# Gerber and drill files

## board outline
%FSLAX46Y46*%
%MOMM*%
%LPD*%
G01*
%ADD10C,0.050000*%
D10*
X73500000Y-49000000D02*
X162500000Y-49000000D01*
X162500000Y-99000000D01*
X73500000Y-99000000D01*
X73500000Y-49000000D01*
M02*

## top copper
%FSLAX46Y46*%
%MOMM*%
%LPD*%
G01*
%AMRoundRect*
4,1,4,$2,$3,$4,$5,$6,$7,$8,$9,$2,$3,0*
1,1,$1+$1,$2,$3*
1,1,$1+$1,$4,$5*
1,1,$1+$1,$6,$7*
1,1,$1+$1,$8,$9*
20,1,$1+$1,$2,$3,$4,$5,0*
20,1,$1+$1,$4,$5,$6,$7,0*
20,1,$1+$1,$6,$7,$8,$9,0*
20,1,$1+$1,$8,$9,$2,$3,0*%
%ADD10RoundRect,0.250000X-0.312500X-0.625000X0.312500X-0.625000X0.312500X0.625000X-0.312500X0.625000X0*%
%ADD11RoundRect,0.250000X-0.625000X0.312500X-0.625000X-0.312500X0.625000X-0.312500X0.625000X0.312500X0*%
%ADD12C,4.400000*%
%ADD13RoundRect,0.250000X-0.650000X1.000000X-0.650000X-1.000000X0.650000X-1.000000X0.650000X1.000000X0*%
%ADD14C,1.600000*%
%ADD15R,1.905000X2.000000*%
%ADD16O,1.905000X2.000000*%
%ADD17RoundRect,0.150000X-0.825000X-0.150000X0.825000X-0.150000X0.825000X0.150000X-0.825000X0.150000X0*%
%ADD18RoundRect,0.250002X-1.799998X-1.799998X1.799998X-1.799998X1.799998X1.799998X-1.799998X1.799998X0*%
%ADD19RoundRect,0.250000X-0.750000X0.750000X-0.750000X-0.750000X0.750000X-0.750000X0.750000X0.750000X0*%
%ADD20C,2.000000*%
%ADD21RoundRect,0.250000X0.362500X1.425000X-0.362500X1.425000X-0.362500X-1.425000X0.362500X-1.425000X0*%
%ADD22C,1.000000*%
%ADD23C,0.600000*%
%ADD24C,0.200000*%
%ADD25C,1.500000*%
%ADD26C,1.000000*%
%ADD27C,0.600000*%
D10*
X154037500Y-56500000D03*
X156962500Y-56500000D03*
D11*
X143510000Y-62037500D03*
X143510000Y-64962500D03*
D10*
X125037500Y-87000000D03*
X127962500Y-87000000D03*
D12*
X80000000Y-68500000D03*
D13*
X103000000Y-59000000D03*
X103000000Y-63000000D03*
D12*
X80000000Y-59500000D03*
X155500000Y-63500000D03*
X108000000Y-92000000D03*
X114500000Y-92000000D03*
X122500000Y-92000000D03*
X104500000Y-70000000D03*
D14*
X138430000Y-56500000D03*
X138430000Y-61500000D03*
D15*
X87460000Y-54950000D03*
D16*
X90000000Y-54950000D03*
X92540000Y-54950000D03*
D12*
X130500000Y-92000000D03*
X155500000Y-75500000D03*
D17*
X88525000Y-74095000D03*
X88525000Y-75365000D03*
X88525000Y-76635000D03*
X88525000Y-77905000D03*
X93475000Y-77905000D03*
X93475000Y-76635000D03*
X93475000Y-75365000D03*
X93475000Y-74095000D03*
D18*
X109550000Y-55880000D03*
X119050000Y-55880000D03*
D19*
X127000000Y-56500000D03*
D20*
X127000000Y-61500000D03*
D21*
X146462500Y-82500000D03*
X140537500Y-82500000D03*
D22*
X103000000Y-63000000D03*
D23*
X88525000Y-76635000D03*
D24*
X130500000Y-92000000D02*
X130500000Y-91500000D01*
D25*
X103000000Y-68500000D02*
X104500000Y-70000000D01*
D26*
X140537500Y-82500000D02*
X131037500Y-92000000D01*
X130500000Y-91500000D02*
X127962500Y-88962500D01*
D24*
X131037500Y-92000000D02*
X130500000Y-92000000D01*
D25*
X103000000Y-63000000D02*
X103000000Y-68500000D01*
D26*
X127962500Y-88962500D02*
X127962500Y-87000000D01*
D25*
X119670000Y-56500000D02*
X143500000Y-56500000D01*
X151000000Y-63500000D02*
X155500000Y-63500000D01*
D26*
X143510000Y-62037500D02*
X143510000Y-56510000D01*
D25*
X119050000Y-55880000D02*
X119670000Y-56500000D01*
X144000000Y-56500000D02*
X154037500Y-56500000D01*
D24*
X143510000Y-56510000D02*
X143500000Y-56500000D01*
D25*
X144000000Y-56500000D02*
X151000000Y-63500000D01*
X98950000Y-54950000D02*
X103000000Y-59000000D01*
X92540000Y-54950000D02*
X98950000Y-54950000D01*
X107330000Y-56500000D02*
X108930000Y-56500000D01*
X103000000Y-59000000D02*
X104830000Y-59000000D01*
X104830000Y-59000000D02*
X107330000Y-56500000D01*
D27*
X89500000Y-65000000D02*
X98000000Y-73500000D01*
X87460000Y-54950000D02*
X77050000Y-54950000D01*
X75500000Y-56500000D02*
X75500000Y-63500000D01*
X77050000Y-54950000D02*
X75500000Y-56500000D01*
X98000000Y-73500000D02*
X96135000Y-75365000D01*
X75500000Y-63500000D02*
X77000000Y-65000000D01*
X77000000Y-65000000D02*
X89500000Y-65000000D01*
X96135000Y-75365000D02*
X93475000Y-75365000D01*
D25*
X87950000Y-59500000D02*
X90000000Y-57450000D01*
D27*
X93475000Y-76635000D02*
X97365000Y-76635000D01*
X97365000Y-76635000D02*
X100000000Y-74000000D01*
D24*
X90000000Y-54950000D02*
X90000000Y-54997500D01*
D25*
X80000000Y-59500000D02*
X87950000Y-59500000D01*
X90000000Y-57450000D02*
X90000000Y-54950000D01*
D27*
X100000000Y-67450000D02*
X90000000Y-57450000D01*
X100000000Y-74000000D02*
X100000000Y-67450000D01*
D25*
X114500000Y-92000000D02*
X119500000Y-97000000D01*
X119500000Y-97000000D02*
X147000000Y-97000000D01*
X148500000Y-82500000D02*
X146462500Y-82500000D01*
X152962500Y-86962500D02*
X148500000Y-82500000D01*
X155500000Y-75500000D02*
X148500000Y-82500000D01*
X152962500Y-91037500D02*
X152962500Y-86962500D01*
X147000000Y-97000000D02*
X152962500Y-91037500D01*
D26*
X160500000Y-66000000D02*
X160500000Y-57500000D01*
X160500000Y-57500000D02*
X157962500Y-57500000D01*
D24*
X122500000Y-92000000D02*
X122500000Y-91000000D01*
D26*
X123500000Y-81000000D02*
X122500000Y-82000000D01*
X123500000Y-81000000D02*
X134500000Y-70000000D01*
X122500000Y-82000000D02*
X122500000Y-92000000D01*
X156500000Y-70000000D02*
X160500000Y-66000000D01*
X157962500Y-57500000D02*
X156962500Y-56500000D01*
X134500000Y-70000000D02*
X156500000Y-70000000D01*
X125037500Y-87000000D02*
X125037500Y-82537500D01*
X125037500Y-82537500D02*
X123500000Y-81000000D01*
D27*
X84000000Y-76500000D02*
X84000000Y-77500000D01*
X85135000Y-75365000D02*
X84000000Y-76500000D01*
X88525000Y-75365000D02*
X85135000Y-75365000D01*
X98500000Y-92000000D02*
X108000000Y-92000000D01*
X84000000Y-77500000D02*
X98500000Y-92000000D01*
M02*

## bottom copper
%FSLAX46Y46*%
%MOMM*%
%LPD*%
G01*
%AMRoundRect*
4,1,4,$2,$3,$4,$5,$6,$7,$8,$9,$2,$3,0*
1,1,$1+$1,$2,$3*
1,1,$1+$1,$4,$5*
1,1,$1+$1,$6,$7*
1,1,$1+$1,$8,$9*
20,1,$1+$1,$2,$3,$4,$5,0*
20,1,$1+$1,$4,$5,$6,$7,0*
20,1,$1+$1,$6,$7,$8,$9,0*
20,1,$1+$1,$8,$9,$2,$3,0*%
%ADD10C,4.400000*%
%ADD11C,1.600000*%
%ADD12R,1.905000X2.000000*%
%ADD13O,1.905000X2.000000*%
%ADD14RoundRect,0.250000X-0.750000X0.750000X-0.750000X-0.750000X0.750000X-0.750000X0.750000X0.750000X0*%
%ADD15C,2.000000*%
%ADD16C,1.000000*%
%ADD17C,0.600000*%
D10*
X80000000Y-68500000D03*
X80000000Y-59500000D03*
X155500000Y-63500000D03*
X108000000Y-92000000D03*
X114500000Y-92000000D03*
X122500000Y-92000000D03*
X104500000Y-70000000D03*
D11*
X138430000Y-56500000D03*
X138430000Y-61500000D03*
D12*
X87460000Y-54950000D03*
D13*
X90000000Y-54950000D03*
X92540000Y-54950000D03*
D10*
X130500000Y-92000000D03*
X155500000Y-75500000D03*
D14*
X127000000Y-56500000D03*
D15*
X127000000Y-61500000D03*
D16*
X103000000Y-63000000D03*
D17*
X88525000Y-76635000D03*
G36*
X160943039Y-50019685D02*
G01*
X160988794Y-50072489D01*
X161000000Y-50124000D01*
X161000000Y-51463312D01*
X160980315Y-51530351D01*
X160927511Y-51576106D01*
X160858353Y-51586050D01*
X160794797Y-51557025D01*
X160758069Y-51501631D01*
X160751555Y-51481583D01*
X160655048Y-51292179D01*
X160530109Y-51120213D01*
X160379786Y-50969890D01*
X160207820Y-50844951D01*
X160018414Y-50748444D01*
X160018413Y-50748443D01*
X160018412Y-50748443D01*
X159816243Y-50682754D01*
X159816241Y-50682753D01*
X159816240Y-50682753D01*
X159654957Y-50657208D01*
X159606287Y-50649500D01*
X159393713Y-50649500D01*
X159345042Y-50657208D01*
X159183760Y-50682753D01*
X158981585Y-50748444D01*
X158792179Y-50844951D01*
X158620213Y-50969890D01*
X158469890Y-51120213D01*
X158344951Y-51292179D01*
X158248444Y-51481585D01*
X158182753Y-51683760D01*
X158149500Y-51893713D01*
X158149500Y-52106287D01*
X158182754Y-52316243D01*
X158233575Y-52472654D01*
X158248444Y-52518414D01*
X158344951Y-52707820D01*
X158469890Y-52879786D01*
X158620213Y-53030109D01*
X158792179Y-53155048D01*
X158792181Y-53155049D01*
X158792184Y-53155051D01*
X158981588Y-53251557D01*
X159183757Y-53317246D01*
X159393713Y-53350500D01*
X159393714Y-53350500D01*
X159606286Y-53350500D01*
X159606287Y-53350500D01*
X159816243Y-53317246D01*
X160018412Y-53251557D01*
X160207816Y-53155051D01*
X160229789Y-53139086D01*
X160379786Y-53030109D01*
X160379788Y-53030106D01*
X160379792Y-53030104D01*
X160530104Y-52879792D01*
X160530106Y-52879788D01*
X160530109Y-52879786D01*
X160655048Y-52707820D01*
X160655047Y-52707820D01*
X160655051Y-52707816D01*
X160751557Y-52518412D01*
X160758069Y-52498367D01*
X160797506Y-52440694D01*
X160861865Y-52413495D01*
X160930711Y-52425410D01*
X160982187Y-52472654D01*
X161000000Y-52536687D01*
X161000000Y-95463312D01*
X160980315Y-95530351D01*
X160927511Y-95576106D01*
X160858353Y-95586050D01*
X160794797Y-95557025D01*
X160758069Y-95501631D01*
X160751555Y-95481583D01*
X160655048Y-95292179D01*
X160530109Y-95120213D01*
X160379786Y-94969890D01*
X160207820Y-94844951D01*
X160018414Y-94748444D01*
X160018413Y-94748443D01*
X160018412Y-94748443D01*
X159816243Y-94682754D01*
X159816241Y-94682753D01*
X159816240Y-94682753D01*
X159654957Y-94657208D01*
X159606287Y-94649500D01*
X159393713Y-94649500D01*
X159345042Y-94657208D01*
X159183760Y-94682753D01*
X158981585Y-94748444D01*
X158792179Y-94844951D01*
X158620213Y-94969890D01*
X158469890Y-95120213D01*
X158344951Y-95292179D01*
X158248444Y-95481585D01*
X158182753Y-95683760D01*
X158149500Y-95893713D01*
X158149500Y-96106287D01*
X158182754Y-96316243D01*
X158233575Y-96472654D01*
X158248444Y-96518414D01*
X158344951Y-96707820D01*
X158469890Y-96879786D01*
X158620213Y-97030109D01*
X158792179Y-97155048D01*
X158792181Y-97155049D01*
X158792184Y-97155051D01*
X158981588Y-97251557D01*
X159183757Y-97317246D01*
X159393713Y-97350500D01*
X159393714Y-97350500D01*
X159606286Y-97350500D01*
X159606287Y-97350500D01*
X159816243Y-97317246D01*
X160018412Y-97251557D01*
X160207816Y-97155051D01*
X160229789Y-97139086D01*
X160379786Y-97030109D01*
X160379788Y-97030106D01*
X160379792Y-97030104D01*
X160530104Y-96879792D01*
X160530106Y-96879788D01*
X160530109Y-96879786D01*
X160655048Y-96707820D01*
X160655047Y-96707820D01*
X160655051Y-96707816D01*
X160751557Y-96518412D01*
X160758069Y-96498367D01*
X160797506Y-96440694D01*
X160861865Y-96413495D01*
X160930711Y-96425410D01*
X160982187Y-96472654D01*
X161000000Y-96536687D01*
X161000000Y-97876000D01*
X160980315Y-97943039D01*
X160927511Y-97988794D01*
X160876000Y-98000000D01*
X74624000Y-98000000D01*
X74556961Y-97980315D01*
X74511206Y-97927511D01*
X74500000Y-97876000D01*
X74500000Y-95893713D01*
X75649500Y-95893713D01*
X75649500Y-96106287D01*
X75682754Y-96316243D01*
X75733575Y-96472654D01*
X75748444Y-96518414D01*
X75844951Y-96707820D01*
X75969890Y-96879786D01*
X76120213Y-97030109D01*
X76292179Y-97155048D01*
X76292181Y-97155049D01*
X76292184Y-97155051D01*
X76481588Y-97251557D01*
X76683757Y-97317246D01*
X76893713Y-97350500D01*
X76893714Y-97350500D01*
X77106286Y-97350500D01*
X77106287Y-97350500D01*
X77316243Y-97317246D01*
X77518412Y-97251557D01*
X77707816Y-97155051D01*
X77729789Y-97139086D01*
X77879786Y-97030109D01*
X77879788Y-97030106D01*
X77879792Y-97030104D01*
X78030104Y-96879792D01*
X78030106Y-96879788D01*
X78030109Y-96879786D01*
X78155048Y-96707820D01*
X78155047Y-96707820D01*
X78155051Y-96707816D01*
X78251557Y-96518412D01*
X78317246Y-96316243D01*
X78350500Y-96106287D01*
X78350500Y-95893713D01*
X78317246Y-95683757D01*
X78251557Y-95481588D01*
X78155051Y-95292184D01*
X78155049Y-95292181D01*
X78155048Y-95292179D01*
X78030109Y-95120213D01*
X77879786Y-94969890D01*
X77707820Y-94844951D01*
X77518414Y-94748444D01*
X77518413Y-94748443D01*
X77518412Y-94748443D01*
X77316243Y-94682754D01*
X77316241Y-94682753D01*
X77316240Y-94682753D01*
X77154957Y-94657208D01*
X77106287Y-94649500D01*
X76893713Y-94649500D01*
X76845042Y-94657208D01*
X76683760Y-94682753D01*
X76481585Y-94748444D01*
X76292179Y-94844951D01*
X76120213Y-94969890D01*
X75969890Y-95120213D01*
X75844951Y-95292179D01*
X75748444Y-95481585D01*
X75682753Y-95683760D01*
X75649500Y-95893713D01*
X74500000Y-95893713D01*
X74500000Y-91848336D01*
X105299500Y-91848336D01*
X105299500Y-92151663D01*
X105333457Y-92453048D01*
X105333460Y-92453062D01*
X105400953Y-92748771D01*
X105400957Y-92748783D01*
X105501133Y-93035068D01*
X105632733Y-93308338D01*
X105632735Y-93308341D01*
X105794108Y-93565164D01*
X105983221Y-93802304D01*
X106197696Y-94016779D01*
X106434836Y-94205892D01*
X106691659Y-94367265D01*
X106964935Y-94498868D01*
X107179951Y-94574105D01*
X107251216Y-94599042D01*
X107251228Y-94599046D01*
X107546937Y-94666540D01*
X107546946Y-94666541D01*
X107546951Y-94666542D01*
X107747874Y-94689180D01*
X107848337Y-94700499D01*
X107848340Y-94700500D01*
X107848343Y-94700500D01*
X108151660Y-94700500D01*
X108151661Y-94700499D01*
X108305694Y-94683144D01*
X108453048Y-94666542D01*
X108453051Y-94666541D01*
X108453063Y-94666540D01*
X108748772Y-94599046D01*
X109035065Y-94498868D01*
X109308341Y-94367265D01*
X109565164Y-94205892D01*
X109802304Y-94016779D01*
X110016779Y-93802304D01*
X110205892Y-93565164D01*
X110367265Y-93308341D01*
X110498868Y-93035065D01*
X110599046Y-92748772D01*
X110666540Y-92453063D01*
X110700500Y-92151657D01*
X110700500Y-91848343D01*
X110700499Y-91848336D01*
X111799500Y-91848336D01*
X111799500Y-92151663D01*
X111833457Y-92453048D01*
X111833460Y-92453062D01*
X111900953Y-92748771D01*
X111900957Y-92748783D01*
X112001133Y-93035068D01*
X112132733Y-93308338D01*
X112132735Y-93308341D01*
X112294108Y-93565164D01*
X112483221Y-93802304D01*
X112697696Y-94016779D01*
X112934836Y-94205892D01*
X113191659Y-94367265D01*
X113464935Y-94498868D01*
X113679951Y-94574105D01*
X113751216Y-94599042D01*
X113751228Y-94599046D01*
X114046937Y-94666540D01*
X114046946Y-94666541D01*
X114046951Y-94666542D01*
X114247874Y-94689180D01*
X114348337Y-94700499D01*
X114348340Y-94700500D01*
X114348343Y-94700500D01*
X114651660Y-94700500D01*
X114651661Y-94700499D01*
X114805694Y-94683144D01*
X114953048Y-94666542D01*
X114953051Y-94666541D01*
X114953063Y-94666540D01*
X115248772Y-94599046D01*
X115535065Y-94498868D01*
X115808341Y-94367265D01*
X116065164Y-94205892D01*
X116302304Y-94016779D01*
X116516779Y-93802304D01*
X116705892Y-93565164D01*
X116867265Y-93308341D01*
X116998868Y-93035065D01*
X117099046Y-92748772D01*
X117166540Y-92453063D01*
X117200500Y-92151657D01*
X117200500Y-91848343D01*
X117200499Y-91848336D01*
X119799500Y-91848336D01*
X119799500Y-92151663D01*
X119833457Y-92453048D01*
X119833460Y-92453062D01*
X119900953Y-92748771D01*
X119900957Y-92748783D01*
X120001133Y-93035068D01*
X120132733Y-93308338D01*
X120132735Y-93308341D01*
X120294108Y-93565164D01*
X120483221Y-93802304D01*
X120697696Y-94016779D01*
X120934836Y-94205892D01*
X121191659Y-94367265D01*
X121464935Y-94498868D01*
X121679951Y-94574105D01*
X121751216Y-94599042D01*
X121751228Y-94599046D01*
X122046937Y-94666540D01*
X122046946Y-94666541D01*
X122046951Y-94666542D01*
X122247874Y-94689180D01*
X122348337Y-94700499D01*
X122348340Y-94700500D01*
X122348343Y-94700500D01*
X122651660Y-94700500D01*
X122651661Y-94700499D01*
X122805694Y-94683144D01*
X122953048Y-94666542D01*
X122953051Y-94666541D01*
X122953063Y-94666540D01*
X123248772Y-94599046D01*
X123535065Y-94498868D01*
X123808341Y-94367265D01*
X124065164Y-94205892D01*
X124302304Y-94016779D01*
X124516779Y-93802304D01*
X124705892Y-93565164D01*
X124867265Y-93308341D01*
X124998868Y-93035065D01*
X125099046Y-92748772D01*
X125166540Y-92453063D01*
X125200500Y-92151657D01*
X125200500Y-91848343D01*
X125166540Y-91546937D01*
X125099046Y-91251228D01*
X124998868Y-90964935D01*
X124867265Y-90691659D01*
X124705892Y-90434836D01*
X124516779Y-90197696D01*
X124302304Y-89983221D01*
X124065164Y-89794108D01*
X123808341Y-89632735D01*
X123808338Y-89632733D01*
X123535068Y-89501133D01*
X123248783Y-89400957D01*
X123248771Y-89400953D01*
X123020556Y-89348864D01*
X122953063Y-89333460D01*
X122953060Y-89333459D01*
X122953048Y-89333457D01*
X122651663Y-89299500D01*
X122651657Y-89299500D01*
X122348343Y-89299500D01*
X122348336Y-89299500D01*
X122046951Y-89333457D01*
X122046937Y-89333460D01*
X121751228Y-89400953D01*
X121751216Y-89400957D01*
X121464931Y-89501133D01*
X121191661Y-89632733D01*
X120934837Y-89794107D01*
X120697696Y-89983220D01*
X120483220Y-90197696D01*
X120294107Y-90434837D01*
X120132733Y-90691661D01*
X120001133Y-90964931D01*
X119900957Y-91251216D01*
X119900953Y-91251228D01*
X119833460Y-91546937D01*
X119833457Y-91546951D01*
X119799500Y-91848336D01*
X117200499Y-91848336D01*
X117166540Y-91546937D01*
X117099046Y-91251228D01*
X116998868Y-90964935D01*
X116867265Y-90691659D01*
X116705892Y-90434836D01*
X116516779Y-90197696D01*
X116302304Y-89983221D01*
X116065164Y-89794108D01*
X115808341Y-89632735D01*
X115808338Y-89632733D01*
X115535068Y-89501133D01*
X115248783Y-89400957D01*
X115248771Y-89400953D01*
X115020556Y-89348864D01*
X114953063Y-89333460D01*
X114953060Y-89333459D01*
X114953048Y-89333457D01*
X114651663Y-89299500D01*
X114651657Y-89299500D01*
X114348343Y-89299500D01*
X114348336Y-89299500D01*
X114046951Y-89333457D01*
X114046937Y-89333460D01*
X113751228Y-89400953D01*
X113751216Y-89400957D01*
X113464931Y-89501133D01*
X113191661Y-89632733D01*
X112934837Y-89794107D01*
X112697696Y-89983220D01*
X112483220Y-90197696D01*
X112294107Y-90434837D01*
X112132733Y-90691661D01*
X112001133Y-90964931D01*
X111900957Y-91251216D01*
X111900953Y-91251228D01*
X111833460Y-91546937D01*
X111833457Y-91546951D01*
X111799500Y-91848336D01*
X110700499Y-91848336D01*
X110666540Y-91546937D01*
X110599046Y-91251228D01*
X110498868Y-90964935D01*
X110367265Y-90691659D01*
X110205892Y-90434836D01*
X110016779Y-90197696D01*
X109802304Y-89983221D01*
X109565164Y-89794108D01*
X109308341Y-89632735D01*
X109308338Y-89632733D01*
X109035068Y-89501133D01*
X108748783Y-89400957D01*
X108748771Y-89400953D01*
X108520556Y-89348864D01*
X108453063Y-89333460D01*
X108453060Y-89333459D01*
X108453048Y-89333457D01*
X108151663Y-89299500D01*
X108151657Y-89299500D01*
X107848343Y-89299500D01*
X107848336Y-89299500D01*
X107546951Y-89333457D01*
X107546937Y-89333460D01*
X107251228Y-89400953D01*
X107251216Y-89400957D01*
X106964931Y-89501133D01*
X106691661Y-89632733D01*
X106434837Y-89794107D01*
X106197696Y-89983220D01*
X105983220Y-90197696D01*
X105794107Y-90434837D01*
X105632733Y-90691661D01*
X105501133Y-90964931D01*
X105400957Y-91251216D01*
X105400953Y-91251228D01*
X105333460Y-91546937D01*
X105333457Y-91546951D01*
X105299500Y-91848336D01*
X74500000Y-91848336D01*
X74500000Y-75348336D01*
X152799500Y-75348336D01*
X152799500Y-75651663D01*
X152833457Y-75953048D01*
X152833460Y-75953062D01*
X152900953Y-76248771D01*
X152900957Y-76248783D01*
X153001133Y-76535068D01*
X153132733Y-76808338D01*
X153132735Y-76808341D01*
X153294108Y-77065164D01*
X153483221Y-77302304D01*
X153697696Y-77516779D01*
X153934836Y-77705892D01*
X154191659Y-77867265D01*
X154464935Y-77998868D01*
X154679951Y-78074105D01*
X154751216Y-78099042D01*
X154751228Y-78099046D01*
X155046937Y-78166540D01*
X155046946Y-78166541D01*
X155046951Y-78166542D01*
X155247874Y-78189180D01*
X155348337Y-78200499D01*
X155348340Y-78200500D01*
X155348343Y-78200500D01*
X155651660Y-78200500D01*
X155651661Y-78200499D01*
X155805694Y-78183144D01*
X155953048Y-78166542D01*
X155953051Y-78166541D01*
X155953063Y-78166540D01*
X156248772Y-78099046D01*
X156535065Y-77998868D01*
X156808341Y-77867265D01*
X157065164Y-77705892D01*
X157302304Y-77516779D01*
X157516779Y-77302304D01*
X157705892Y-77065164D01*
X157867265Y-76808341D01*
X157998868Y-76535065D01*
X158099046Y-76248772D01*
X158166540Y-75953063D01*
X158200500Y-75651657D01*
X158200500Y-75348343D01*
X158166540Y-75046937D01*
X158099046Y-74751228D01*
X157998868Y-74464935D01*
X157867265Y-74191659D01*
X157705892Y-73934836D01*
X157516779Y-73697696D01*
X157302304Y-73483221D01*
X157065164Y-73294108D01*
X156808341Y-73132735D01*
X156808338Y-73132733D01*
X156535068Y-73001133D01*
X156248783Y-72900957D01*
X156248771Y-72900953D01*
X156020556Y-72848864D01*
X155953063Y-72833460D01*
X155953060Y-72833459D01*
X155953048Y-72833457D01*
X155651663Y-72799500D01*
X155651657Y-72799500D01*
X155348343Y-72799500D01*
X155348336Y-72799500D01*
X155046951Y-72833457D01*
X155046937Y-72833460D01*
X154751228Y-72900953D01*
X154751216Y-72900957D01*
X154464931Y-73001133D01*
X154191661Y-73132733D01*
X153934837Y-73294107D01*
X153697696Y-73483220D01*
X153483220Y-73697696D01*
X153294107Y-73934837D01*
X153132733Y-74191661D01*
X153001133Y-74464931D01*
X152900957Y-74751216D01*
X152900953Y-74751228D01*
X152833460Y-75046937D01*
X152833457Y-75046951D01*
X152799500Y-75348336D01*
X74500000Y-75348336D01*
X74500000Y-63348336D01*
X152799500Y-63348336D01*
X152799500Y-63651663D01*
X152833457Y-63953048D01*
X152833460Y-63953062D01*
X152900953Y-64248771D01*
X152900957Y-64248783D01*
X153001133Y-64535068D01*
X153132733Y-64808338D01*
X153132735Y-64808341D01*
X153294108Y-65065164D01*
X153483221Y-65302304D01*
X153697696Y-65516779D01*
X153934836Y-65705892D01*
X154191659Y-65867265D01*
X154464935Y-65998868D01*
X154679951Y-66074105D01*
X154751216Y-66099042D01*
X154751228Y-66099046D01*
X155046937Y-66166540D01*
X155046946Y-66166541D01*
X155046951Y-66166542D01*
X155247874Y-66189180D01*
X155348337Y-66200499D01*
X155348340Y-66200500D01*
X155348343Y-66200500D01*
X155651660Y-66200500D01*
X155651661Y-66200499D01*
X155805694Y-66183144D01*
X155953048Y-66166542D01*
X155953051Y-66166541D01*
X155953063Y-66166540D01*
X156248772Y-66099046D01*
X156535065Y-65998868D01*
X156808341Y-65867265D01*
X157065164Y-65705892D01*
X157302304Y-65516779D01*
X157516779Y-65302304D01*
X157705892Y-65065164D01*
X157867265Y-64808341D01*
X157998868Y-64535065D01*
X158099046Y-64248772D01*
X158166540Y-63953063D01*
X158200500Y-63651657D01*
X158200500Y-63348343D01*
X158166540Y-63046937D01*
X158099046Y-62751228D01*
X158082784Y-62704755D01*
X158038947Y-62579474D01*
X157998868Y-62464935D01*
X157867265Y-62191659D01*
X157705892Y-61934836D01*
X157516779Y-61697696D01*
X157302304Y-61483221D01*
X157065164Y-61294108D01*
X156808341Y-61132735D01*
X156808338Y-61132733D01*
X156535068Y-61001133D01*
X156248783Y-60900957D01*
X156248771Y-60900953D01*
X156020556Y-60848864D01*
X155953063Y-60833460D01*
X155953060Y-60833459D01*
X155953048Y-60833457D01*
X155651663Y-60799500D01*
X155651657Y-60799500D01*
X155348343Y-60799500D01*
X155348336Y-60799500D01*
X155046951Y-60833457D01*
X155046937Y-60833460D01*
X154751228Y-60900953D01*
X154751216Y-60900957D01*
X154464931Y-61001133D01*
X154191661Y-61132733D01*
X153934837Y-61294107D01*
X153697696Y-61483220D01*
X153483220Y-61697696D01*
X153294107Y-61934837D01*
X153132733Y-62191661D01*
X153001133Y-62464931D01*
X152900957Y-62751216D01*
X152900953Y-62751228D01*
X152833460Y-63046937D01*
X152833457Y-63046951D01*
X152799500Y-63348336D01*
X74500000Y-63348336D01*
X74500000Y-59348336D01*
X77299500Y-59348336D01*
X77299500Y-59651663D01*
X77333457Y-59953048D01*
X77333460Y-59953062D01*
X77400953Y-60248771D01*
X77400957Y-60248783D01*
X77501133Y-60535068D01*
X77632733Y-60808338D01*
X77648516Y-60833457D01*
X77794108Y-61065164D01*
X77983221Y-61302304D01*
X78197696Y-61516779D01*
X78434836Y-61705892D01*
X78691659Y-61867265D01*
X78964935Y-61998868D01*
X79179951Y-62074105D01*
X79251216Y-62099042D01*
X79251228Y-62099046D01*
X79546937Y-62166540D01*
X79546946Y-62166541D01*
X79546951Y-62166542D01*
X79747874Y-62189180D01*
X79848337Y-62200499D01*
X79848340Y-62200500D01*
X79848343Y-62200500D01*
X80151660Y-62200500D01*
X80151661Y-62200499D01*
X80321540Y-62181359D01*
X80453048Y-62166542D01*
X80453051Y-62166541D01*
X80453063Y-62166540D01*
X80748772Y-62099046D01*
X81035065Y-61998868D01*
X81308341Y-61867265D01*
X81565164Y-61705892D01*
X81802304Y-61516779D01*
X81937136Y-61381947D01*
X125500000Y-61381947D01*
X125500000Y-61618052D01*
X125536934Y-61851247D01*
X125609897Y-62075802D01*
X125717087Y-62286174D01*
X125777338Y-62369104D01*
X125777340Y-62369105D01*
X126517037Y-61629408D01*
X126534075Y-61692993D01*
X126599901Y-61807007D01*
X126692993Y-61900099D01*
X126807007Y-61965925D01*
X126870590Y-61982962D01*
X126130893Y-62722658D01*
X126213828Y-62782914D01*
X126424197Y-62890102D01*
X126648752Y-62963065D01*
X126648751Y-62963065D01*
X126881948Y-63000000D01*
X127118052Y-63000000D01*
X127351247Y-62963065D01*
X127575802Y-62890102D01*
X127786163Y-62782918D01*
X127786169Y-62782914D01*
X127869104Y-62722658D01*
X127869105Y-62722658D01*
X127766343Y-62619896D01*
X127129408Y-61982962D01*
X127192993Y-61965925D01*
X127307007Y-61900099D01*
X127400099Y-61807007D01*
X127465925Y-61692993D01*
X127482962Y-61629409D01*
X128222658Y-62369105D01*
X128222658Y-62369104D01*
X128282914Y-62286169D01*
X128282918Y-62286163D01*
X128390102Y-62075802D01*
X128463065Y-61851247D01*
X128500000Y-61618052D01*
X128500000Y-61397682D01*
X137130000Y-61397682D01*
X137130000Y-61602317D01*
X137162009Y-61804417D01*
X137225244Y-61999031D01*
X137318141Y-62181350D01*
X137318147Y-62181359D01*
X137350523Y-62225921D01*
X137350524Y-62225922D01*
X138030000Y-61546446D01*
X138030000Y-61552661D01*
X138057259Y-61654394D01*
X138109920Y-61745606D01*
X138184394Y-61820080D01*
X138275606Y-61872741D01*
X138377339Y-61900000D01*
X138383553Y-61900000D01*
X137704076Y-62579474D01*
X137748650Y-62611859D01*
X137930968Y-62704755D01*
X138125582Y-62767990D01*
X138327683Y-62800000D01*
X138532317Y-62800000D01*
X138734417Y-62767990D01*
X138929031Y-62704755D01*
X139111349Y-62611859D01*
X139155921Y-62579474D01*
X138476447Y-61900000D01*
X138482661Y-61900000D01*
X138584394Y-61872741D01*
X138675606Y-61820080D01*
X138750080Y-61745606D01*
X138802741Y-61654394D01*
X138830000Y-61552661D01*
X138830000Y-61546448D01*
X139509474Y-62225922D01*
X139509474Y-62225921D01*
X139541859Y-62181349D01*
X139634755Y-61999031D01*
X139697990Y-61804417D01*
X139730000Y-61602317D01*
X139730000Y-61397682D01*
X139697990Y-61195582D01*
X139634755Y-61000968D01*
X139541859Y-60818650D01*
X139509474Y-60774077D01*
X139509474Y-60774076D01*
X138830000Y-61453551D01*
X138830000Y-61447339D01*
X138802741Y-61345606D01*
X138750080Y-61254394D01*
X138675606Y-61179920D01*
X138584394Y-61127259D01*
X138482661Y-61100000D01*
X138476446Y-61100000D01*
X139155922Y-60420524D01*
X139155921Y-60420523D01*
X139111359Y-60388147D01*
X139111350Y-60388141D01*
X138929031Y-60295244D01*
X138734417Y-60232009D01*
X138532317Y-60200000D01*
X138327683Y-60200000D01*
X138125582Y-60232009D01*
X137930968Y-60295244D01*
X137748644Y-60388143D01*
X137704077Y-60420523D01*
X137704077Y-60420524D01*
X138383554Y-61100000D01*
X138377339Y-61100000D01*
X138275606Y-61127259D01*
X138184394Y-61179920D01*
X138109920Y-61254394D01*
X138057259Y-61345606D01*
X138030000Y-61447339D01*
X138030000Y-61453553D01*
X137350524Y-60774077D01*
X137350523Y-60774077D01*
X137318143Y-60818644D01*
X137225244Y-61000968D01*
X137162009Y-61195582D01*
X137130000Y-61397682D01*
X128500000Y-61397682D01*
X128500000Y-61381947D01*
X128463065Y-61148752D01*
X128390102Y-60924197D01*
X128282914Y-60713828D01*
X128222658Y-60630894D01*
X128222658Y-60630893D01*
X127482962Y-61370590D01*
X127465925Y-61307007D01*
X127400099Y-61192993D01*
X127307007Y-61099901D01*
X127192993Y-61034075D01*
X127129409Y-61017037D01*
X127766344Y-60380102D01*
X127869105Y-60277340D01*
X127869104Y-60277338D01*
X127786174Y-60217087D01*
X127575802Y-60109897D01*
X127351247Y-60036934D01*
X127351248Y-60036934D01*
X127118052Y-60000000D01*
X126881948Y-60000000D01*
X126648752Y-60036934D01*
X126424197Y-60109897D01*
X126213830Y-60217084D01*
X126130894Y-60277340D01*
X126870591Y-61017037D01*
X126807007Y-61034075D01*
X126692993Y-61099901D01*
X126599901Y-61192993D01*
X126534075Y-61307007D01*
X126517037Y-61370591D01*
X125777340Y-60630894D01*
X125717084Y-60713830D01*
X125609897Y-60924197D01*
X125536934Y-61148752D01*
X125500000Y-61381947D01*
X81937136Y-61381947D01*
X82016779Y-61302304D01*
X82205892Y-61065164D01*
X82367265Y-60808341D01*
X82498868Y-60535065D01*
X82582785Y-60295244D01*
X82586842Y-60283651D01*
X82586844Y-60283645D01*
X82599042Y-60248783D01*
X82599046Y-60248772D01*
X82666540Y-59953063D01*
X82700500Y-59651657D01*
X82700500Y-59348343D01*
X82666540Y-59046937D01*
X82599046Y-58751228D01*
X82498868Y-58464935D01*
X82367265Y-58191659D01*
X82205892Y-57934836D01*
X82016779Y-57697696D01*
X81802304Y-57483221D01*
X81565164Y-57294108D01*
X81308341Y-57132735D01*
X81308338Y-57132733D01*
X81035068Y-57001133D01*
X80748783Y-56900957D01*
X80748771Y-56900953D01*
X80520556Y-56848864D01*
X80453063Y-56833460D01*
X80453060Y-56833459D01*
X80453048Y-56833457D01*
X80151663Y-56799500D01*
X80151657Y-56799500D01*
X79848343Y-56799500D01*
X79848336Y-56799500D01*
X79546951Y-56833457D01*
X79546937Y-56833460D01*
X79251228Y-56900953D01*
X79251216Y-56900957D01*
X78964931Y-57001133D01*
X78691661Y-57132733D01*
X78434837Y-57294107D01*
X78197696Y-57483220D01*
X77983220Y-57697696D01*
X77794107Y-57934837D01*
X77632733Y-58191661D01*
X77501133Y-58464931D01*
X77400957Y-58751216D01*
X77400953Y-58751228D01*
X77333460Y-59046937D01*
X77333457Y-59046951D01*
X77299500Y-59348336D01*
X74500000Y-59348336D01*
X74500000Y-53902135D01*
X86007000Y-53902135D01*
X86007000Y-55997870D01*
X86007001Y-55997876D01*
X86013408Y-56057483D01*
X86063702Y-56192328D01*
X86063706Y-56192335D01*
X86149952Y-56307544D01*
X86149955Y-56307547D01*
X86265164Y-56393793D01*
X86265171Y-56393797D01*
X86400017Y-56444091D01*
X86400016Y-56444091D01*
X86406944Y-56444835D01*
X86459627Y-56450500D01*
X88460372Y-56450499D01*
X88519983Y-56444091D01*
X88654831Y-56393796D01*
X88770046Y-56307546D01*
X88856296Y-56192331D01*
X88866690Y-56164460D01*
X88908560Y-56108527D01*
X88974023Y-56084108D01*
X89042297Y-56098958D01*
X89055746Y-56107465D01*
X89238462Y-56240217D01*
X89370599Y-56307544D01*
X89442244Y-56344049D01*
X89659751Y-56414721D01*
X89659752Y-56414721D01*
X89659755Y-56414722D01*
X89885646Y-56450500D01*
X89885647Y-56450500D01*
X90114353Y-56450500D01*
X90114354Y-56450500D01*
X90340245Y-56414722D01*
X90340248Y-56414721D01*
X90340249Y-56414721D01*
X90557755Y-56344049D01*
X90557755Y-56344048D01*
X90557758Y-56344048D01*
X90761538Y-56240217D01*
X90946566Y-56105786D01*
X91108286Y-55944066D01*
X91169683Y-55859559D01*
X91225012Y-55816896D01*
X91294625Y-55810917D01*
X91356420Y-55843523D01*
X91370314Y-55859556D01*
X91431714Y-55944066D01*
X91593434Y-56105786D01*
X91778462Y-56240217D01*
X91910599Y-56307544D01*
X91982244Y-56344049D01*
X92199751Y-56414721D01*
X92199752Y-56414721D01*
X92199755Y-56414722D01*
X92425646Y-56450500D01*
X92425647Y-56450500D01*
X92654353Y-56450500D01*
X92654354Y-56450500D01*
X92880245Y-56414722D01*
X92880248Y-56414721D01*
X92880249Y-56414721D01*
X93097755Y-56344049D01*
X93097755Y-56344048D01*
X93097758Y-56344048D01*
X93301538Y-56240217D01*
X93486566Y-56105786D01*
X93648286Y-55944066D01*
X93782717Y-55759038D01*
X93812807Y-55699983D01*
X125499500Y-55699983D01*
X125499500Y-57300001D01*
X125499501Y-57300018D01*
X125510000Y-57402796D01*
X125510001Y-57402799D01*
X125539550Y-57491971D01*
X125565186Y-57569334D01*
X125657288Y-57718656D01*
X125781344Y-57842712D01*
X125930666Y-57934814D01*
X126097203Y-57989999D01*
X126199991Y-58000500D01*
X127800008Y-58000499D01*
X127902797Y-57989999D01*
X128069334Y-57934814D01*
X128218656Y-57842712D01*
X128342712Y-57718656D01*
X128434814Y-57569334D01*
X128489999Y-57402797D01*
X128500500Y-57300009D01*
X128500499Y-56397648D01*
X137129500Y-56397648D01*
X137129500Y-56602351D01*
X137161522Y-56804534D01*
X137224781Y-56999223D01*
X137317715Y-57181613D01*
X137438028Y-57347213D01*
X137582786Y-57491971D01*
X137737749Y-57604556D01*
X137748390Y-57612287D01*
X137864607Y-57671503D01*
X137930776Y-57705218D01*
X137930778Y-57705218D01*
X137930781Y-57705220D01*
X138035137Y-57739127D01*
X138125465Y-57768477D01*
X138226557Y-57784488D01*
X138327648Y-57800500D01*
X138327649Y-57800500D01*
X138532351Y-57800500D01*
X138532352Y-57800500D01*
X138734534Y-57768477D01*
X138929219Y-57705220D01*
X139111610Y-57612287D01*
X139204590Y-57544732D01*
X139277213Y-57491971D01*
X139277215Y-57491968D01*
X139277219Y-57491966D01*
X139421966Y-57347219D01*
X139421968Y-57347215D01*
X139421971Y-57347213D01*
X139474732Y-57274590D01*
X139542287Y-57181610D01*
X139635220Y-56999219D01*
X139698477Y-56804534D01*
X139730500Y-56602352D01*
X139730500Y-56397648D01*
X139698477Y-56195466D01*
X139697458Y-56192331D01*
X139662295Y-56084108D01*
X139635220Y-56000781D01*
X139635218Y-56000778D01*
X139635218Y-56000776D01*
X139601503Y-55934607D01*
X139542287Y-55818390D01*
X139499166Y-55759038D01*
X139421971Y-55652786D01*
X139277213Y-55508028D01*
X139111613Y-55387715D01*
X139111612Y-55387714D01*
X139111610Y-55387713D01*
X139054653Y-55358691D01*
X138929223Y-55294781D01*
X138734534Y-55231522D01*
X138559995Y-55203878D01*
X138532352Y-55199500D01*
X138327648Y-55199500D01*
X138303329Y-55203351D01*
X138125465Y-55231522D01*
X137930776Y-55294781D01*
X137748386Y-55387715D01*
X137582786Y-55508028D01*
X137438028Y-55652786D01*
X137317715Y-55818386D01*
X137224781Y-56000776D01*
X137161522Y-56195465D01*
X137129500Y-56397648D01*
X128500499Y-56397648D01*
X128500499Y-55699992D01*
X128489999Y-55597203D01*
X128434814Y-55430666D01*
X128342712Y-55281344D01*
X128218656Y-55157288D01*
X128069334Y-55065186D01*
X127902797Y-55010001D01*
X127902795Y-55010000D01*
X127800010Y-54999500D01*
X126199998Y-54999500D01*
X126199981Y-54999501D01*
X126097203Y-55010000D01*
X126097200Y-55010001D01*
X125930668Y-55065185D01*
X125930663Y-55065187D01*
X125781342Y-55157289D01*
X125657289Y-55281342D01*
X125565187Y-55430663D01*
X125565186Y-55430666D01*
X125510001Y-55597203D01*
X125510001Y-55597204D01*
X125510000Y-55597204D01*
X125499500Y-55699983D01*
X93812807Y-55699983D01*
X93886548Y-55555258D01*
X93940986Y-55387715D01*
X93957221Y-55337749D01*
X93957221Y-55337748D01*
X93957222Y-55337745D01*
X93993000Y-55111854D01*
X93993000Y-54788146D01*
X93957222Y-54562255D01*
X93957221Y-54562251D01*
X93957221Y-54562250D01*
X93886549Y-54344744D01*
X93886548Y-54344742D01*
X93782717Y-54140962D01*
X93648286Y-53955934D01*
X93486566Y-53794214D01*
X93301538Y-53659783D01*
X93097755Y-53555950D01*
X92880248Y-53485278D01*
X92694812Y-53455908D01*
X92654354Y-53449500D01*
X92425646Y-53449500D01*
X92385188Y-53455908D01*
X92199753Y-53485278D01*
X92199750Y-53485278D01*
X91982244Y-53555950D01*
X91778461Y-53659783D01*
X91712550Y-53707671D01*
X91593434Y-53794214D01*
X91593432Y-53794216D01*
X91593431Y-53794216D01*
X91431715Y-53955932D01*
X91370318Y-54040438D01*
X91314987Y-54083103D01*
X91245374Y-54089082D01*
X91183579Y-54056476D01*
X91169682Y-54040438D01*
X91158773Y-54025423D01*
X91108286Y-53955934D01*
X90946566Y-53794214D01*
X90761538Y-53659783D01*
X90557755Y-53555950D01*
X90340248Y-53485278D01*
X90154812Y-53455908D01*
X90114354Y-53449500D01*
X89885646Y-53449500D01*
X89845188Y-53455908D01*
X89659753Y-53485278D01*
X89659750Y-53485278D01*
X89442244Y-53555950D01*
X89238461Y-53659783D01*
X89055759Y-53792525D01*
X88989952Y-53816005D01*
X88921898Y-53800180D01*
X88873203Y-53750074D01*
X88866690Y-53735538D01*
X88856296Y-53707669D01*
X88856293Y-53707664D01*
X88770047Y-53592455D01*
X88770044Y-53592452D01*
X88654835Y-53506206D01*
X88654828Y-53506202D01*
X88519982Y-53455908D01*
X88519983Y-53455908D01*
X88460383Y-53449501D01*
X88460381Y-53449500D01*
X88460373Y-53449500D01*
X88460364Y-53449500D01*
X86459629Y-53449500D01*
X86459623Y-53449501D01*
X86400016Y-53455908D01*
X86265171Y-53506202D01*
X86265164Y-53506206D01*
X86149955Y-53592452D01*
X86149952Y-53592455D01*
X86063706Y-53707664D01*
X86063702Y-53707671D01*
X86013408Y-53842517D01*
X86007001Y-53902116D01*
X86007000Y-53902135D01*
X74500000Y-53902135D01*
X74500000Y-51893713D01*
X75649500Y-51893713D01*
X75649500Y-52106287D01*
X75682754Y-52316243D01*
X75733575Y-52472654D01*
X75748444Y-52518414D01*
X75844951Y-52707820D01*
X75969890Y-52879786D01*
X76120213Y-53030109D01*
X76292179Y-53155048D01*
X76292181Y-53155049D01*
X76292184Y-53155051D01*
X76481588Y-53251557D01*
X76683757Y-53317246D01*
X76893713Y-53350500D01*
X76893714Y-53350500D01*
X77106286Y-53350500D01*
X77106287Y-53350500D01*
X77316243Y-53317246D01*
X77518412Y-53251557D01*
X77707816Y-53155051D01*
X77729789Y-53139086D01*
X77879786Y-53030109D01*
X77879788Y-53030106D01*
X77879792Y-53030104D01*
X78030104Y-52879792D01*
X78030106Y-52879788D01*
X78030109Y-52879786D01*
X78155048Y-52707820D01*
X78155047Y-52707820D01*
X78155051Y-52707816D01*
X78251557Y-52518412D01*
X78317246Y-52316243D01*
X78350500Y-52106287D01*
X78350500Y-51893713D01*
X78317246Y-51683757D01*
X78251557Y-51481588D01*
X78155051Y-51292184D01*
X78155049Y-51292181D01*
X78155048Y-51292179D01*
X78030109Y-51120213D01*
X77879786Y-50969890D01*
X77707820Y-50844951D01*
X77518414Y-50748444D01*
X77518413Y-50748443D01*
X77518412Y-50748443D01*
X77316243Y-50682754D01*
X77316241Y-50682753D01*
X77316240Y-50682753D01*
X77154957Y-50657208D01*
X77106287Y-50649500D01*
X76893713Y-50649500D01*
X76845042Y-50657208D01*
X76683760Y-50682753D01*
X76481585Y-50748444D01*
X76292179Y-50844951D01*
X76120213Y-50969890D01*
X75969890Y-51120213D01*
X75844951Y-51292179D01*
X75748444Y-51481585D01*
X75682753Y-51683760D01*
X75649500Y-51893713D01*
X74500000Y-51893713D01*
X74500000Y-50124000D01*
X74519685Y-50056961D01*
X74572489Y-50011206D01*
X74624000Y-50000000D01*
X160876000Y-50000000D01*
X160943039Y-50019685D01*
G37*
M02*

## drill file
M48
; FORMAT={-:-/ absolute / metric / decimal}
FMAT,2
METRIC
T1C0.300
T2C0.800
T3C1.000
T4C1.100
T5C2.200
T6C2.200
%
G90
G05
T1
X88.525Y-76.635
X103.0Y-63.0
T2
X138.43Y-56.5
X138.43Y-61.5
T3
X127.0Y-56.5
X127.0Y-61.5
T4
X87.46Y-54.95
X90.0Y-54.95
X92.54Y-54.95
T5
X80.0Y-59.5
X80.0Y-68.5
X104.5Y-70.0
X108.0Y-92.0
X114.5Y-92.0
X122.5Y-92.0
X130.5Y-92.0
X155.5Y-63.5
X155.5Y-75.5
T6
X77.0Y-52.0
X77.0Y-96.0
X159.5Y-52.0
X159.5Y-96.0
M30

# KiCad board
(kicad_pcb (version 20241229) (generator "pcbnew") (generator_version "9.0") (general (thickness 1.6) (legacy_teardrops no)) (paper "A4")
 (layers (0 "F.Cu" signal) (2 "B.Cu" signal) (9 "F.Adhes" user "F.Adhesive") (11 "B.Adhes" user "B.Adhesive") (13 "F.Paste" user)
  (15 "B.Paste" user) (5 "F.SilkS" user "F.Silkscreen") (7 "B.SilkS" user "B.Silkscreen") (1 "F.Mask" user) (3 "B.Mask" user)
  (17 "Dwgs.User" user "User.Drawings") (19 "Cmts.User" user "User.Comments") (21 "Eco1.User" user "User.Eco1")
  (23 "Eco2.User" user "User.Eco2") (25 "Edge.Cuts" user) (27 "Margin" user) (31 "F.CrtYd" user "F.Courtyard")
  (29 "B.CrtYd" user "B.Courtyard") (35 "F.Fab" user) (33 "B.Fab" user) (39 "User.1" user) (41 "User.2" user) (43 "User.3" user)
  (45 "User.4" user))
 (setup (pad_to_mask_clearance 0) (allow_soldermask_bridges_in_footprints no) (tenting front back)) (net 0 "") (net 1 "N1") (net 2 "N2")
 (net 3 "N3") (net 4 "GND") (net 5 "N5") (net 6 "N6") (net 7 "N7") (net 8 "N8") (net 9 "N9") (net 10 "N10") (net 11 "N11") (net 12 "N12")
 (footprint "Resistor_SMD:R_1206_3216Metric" (layer "F.Cu") (at 155.5 56.5)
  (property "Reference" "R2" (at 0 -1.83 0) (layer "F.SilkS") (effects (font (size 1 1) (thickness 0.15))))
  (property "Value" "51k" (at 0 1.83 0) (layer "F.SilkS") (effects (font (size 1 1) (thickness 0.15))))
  (pad "1" smd roundrect (at -1.4625 0) (size 1.125 1.75) (layers "F.Cu" "F.Mask" "F.Paste") (roundrect_rratio 0.222222) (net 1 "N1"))
  (pad "2" smd roundrect (at 1.4625 0) (size 1.125 1.75) (layers "F.Cu" "F.Mask" "F.Paste") (roundrect_rratio 0.222222) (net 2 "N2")))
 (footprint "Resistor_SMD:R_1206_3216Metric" (layer "F.Cu") (at 143.51 63.5 -90)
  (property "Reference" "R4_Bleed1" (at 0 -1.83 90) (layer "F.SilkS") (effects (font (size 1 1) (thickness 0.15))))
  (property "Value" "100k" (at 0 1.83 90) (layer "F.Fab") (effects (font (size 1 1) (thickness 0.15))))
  (pad "1" smd roundrect (at -1.4625 0 270) (size 1.125 1.75) (layers "F.Cu" "F.Mask" "F.Paste") (roundrect_rratio 0.222222) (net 1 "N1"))
  (pad "2" smd roundrect (at 1.4625 0 270) (size 1.125 1.75) (layers "F.Cu" "F.Mask" "F.Paste") (roundrect_rratio 0.222222) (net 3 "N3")))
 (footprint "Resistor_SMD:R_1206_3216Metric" (layer "F.Cu") (at 126.5 87)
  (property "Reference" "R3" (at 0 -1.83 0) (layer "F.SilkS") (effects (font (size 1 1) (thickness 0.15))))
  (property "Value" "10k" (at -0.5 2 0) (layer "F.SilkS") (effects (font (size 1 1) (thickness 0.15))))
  (pad "1" smd roundrect (at -1.4625 0) (size 1.125 1.75) (layers "F.Cu" "F.Mask" "F.Paste") (roundrect_rratio 0.222222) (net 2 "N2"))
  (pad "2" smd roundrect (at 1.4625 0) (size 1.125 1.75) (layers "F.Cu" "F.Mask" "F.Paste") (roundrect_rratio 0.222222) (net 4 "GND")))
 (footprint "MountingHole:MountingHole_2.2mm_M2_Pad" (layer "F.Cu") (at 80 68.5)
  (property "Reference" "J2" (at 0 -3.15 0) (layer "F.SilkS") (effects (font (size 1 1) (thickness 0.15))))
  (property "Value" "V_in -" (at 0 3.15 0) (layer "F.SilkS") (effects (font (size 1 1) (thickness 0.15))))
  (pad "1" thru_hole circle (at 0 0) (size 4.4 4.4) (drill 2.2) (layers "*.Cu" "*.Mask") (remove_unused_layers no) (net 4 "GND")
   (zone_connect 2)))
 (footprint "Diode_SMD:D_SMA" (layer "F.Cu") (at 103 61 -90)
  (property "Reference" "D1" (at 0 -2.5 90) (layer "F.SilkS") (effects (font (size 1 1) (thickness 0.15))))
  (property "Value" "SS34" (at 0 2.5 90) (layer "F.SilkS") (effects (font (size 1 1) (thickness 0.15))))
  (pad "1" smd roundrect (at -2 0 270) (size 2.5 1.8) (layers "F.Cu" "F.Mask" "F.Paste") (roundrect_rratio 0.1388888889) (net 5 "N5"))
  (pad "2" smd roundrect (at 2 0 270) (size 2.5 1.8) (layers "F.Cu" "F.Mask" "F.Paste") (roundrect_rratio 0.1388888889) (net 4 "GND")))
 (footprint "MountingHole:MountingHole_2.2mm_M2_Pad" (layer "F.Cu") (at 80 59.5)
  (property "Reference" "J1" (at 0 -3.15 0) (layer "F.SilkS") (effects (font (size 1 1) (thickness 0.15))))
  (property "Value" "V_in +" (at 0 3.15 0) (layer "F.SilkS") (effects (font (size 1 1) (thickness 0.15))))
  (pad "1" thru_hole circle (at 0 0) (size 4.4 4.4) (drill 2.2) (layers "*.Cu" "*.Mask") (remove_unused_layers no) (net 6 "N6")
   (zone_connect 2)))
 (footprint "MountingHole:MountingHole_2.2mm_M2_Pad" (layer "F.Cu") (at 155.5 63.5)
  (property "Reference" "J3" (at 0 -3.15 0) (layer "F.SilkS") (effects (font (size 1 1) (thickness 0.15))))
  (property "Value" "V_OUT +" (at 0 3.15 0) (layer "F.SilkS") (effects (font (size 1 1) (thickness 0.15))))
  (pad "1" thru_hole circle (at 0 0) (size 4.4 4.4) (drill 2.2) (layers "*.Cu" "*.Mask") (remove_unused_layers no) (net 1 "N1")
   (zone_connect 2)))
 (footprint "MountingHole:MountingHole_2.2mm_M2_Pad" (layer "F.Cu") (at 108 92)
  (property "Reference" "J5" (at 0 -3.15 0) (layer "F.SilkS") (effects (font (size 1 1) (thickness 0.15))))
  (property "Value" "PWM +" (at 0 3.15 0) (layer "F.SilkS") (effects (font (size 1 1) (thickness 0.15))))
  (pad "1" thru_hole circle (at 0 0) (size 4.4 4.4) (drill 2.2) (layers "*.Cu" "*.Mask") (remove_unused_layers no) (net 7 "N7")
   (zone_connect 2)))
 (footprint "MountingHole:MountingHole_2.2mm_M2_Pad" (layer "F.Cu") (at 114.5 92)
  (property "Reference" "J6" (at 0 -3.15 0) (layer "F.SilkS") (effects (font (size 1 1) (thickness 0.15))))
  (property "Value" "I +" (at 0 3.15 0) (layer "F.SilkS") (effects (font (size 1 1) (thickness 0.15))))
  (pad "1" thru_hole circle (at 0 0) (size 4.4 4.4) (drill 2.2) (layers "*.Cu" "*.Mask") (remove_unused_layers no) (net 3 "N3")
   (zone_connect 2)))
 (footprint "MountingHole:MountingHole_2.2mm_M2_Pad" (layer "F.Cu") (at 122.5 92)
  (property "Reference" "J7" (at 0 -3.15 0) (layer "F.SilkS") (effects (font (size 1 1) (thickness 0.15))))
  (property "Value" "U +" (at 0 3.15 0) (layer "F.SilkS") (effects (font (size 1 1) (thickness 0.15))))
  (pad "1" thru_hole circle (at 0 0) (size 4.4 4.4) (drill 2.2) (layers "*.Cu" "*.Mask") (remove_unused_layers no) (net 2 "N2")
   (zone_connect 2)))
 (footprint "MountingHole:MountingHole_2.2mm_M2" (layer "F.Cu") (at 159.5 52)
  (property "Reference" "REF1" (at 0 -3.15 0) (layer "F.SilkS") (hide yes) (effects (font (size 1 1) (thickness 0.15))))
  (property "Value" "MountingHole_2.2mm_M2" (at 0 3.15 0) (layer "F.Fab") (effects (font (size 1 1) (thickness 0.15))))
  (pad "" np_thru_hole circle (at 0 0) (size 2.2 2.2) (drill 2.2) (layers "*.Cu" "*.Mask")))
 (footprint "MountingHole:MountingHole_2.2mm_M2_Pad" (layer "F.Cu") (at 104.5 70 180)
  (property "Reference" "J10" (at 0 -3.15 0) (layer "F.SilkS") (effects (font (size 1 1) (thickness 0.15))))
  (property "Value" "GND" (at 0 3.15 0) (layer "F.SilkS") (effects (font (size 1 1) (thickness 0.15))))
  (pad "1" thru_hole circle (at 0 0 180) (size 4.4 4.4) (drill 2.2) (layers "*.Cu" "*.Mask") (remove_unused_layers no) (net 4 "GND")
   (zone_connect 2)))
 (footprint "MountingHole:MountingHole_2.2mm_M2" (layer "F.Cu") (at 77 52)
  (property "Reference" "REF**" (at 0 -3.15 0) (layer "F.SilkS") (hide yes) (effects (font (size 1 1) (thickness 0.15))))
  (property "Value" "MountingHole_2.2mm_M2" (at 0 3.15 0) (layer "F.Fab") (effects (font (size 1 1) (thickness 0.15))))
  (pad "" np_thru_hole circle (at 0 0) (size 2.2 2.2) (drill 2.2) (layers "*.Cu" "*.Mask")))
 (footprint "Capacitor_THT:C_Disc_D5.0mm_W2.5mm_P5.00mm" (layer "F.Cu") (at 138.43 56.5 -90)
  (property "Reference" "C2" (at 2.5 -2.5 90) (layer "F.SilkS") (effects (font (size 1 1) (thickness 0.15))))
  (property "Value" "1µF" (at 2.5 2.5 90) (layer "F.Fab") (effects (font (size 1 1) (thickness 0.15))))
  (pad "1" thru_hole circle (at 0 0 270) (size 1.6 1.6) (drill 0.8) (layers "*.Cu" "*.Mask") (remove_unused_layers no) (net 1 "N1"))
  (pad "2" thru_hole circle (at 5 0 270) (size 1.6 1.6) (drill 0.8) (layers "*.Cu" "*.Mask") (remove_unused_layers no) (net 4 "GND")))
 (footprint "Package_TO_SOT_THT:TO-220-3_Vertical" (layer "F.Cu") (at 87.46 54.95)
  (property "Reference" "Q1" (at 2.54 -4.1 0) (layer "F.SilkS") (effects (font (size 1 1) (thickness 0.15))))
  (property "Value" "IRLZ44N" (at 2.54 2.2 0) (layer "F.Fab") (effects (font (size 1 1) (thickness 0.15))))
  (pad "1" thru_hole rect (at 0 0) (size 1.905 2) (drill 1.1) (layers "*.Cu" "*.Mask") (remove_unused_layers no) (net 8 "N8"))
  (pad "2" thru_hole oval (at 2.54 0) (size 1.905 2) (drill 1.1) (layers "*.Cu" "*.Mask") (remove_unused_layers no) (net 6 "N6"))
  (pad "3" thru_hole oval (at 5.08 0) (size 1.905 2) (drill 1.1) (layers "*.Cu" "*.Mask") (remove_unused_layers no) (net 5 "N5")))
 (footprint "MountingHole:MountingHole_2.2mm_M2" (layer "F.Cu") (at 77 96)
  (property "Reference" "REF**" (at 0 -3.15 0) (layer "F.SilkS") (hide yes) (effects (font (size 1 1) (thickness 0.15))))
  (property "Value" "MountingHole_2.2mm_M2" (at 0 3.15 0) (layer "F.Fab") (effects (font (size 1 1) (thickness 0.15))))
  (pad "" np_thru_hole circle (at 0 0) (size 2.2 2.2) (drill 2.2) (layers "*.Cu" "*.Mask")))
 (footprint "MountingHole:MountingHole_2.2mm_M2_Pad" (layer "F.Cu") (at 130.5 92)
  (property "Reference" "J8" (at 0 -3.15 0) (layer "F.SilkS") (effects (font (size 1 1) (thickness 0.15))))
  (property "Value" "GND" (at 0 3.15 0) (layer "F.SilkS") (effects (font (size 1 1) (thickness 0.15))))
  (pad "1" thru_hole circle (at 0 0) (size 4.4 4.4) (drill 2.2) (layers "*.Cu" "*.Mask") (remove_unused_layers no) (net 4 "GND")
   (zone_connect 2)))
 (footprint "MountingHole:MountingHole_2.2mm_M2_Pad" (layer "F.Cu") (at 155.5 75.5)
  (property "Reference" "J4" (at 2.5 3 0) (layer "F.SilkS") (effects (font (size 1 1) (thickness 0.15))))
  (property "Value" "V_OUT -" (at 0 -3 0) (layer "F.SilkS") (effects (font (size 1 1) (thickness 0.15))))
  (pad "1" thru_hole circle (at 0 0) (size 4.4 4.4) (drill 2.2) (layers "*.Cu" "*.Mask") (remove_unused_layers no) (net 3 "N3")
   (zone_connect 2)))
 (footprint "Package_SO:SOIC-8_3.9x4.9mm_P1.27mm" (layer "F.Cu") (at 91 76)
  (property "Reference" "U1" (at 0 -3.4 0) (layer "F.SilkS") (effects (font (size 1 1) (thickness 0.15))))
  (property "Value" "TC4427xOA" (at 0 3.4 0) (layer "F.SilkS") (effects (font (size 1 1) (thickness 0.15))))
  (pad "1" smd roundrect (at -2.475 -1.905) (size 1.95 0.6) (layers "F.Cu" "F.Mask" "F.Paste") (roundrect_rratio 0.25) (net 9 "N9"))
  (pad "2" smd roundrect (at -2.475 -0.635) (size 1.95 0.6) (layers "F.Cu" "F.Mask" "F.Paste") (roundrect_rratio 0.25) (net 7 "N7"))
  (pad "3" smd roundrect (at -2.475 0.635) (size 1.95 0.6) (layers "F.Cu" "F.Mask" "F.Paste") (roundrect_rratio 0.25) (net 4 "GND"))
  (pad "4" smd roundrect (at -2.475 1.905) (size 1.95 0.6) (layers "F.Cu" "F.Mask" "F.Paste") (roundrect_rratio 0.25) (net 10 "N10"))
  (pad "5" smd roundrect (at 2.475 1.905) (size 1.95 0.6) (layers "F.Cu" "F.Mask" "F.Paste") (roundrect_rratio 0.25) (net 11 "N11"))
  (pad "6" smd roundrect (at 2.475 0.635) (size 1.95 0.6) (layers "F.Cu" "F.Mask" "F.Paste") (roundrect_rratio 0.25) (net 6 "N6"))
  (pad "7" smd roundrect (at 2.475 -0.635) (size 1.95 0.6) (layers "F.Cu" "F.Mask" "F.Paste") (roundrect_rratio 0.25) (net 8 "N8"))
  (pad "8" smd roundrect (at 2.475 -1.905) (size 1.95 0.6) (layers "F.Cu" "F.Mask" "F.Paste") (roundrect_rratio 0.25) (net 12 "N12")))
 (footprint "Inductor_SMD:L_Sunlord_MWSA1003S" (layer "F.Cu") (at 114.3 55.88)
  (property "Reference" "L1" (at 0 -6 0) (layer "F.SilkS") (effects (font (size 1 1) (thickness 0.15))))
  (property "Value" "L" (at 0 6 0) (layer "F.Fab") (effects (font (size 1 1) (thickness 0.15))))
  (pad "1" smd roundrect (at -4.75 0) (size 4.1 4.1) (layers "F.Cu" "F.Mask" "F.Paste") (roundrect_rratio 0.060976) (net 5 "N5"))
  (pad "2" smd roundrect (at 4.75 0) (size 4.1 4.1) (layers "F.Cu" "F.Mask" "F.Paste") (roundrect_rratio 0.060976) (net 1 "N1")))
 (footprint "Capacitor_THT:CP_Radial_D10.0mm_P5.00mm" (layer "F.Cu") (at 127 56.5 -90)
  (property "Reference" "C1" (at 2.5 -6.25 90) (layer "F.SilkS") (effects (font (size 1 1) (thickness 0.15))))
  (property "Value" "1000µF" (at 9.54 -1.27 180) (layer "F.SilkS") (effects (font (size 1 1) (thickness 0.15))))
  (pad "1" thru_hole roundrect (at 0 0 270) (size 2 2) (drill 1) (layers "*.Cu" "*.Mask") (remove_unused_layers no) (roundrect_rratio 0.125)
   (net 1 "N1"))
  (pad "2" thru_hole circle (at 5 0 270) (size 2 2) (drill 1) (layers "*.Cu" "*.Mask") (remove_unused_layers no) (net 4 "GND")))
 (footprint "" (layer "F.Cu") (at 159.5 96)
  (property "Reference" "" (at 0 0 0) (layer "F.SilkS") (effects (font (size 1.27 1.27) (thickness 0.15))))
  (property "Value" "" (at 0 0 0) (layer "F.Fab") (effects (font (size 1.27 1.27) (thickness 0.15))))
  (pad "" np_thru_hole circle (at 0 0) (size 2.2 2.2) (drill 2.2) (layers "*.Cu" "*.Mask")))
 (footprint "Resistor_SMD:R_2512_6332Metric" (layer "F.Cu") (at 143.5 82.5 180)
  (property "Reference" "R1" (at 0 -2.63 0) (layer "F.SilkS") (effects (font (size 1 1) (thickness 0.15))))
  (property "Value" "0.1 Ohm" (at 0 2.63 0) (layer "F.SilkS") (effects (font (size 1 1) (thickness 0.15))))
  (pad "1" smd roundrect (at -2.9625 0 180) (size 1.225 3.35) (layers "F.Cu" "F.Mask" "F.Paste") (roundrect_rratio 0.204082) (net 3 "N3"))
  (pad "2" smd roundrect (at 2.9625 0 180) (size 1.225 3.35) (layers "F.Cu" "F.Mask" "F.Paste") (roundrect_rratio 0.204082) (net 4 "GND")))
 (gr_rect (start 73.5 49) (end 162.5 99) (stroke (width 0.05) (type default)) (fill no) (layer "Edge.Cuts"))
 (segment (start 130.5 92) (end 130.5 91.5) (width 0.2) (layer "F.Cu") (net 4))
 (segment (start 103 68.5) (end 104.5 70) (width 1.5) (layer "F.Cu") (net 4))
 (segment (start 140.5375 82.5) (end 131.0375 92) (width 1) (layer "F.Cu") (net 4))
 (segment (start 130.5 91.5) (end 127.9625 88.9625) (width 1) (layer "F.Cu") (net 4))
 (segment (start 131.0375 92) (end 130.5 92) (width 0.2) (layer "F.Cu") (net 4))
 (segment (start 103 63) (end 103 68.5) (width 1.5) (layer "F.Cu") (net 4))
 (segment (start 127.9625 88.9625) (end 127.9625 87) (width 1) (layer "F.Cu") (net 4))
 (via (at 103 63) (size 1) (drill 0.3) (layers "F.Cu" "B.Cu") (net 4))
 (via (at 88.525 76.635) (size 0.6) (drill 0.3) (layers "F.Cu" "B.Cu") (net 4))
 (segment (start 119.67 56.5) (end 143.5 56.5) (width 1.5) (layer "F.Cu") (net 1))
 (segment (start 151 63.5) (end 155.5 63.5) (width 1.5) (layer "F.Cu") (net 1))
 (segment (start 143.51 62.0375) (end 143.51 56.51) (width 1) (layer "F.Cu") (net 1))
 (segment (start 119.05 55.88) (end 119.67 56.5) (width 1.5) (layer "F.Cu") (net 1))
 (segment (start 144 56.5) (end 154.0375 56.5) (width 1.5) (layer "F.Cu") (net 1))
 (segment (start 143.51 56.51) (end 143.5 56.5) (width 0.2) (layer "F.Cu") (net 1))
 (segment (start 144 56.5) (end 151 63.5) (width 1.5) (layer "F.Cu") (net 1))
 (segment (start 98.95 54.95) (end 103 59) (width 1.5) (layer "F.Cu") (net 5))
 (segment (start 92.54 54.95) (end 98.95 54.95) (width 1.5) (layer "F.Cu") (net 5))
 (segment (start 107.33 56.5) (end 108.93 56.5) (width 1.5) (layer "F.Cu") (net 5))
 (segment (start 103 59) (end 104.83 59) (width 1.5) (layer "F.Cu") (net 5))
 (segment (start 104.83 59) (end 107.33 56.5) (width 1.5) (layer "F.Cu") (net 5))
 (segment (start 89.5 65) (end 98 73.5) (width 0.6) (layer "F.Cu") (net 8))
 (segment (start 87.46 54.95) (end 77.05 54.95) (width 0.6) (layer "F.Cu") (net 8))
 (segment (start 75.5 56.5) (end 75.5 63.5) (width 0.6) (layer "F.Cu") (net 8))
 (segment (start 77.05 54.95) (end 75.5 56.5) (width 0.6) (layer "F.Cu") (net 8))
 (segment (start 98 73.5) (end 96.135 75.365) (width 0.6) (layer "F.Cu") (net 8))
 (segment (start 75.5 63.5) (end 77 65) (width 0.6) (layer "F.Cu") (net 8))
 (segment (start 77 65) (end 89.5 65) (width 0.6) (layer "F.Cu") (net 8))
 (segment (start 96.135 75.365) (end 93.475 75.365) (width 0.6) (layer "F.Cu") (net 8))
 (segment (start 87.95 59.5) (end 90 57.45) (width 1.5) (layer "F.Cu") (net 6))
 (segment (start 93.475 76.635) (end 97.365 76.635) (width 0.6) (layer "F.Cu") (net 6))
 (segment (start 97.365 76.635) (end 100 74) (width 0.6) (layer "F.Cu") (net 6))
 (segment (start 90 54.95) (end 90 54.9975) (width 0.2) (layer "F.Cu") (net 6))
 (segment (start 80 59.5) (end 87.95 59.5) (width 1.5) (layer "F.Cu") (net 6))
 (segment (start 90 57.45) (end 90 54.95) (width 1.5) (layer "F.Cu") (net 6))
 (segment (start 100 67.45) (end 90 57.45) (width 0.6) (layer "F.Cu") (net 6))
 (segment (start 100 74) (end 100 67.45) (width 0.6) (layer "F.Cu") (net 6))
 (segment (start 114.5 92) (end 119.5 97) (width 1.5) (layer "F.Cu") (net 3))
 (segment (start 119.5 97) (end 147 97) (width 1.5) (layer "F.Cu") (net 3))
 (segment (start 148.5 82.5) (end 146.4625 82.5) (width 1.5) (layer "F.Cu") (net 3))
 (segment (start 152.9625 86.9625) (end 148.5 82.5) (width 1.5) (layer "F.Cu") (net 3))
 (segment (start 155.5 75.5) (end 148.5 82.5) (width 1.5) (layer "F.Cu") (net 3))
 (segment (start 152.9625 91.0375) (end 152.9625 86.9625) (width 1.5) (layer "F.Cu") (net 3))
 (segment (start 147 97) (end 152.9625 91.0375) (width 1.5) (layer "F.Cu") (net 3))
 (segment (start 160.5 66) (end 160.5 57.5) (width 1) (layer "F.Cu") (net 2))
 (segment (start 160.5 57.5) (end 157.9625 57.5) (width 1) (layer "F.Cu") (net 2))
 (segment (start 122.5 92) (end 122.5 91) (width 0.2) (layer "F.Cu") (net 2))
 (segment (start 123.5 81) (end 122.5 82) (width 1) (layer "F.Cu") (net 2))
 (segment (start 123.5 81) (end 134.5 70) (width 1) (layer "F.Cu") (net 2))
 (segment (start 122.5 82) (end 122.5 92) (width 1) (layer "F.Cu") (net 2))
 (segment (start 156.5 70) (end 160.5 66) (width 1) (layer "F.Cu") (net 2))
 (segment (start 157.9625 57.5) (end 156.9625 56.5) (width 1) (layer "F.Cu") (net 2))
 (segment (start 134.5 70) (end 156.5 70) (width 1) (layer "F.Cu") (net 2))
 (segment (start 125.0375 87) (end 125.0375 82.5375) (width 1) (layer "F.Cu") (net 2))
 (segment (start 125.0375 82.5375) (end 123.5 81) (width 1) (layer "F.Cu") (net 2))
 (segment (start 84 76.5) (end 84 77.5) (width 0.6) (layer "F.Cu") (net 7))
 (segment (start 85.135 75.365) (end 84 76.5) (width 0.6) (layer "F.Cu") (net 7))
 (segment (start 88.525 75.365) (end 85.135 75.365) (width 0.6) (layer "F.Cu") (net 7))
 (segment (start 98.5 92) (end 108 92) (width 0.6) (layer "F.Cu") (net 7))
 (segment (start 84 77.5) (end 98.5 92) (width 0.6) (layer "F.Cu") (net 7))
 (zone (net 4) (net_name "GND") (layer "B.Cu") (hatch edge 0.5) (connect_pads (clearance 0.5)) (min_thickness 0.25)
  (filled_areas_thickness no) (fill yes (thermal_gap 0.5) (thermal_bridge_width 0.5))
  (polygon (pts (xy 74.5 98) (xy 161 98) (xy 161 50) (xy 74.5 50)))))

